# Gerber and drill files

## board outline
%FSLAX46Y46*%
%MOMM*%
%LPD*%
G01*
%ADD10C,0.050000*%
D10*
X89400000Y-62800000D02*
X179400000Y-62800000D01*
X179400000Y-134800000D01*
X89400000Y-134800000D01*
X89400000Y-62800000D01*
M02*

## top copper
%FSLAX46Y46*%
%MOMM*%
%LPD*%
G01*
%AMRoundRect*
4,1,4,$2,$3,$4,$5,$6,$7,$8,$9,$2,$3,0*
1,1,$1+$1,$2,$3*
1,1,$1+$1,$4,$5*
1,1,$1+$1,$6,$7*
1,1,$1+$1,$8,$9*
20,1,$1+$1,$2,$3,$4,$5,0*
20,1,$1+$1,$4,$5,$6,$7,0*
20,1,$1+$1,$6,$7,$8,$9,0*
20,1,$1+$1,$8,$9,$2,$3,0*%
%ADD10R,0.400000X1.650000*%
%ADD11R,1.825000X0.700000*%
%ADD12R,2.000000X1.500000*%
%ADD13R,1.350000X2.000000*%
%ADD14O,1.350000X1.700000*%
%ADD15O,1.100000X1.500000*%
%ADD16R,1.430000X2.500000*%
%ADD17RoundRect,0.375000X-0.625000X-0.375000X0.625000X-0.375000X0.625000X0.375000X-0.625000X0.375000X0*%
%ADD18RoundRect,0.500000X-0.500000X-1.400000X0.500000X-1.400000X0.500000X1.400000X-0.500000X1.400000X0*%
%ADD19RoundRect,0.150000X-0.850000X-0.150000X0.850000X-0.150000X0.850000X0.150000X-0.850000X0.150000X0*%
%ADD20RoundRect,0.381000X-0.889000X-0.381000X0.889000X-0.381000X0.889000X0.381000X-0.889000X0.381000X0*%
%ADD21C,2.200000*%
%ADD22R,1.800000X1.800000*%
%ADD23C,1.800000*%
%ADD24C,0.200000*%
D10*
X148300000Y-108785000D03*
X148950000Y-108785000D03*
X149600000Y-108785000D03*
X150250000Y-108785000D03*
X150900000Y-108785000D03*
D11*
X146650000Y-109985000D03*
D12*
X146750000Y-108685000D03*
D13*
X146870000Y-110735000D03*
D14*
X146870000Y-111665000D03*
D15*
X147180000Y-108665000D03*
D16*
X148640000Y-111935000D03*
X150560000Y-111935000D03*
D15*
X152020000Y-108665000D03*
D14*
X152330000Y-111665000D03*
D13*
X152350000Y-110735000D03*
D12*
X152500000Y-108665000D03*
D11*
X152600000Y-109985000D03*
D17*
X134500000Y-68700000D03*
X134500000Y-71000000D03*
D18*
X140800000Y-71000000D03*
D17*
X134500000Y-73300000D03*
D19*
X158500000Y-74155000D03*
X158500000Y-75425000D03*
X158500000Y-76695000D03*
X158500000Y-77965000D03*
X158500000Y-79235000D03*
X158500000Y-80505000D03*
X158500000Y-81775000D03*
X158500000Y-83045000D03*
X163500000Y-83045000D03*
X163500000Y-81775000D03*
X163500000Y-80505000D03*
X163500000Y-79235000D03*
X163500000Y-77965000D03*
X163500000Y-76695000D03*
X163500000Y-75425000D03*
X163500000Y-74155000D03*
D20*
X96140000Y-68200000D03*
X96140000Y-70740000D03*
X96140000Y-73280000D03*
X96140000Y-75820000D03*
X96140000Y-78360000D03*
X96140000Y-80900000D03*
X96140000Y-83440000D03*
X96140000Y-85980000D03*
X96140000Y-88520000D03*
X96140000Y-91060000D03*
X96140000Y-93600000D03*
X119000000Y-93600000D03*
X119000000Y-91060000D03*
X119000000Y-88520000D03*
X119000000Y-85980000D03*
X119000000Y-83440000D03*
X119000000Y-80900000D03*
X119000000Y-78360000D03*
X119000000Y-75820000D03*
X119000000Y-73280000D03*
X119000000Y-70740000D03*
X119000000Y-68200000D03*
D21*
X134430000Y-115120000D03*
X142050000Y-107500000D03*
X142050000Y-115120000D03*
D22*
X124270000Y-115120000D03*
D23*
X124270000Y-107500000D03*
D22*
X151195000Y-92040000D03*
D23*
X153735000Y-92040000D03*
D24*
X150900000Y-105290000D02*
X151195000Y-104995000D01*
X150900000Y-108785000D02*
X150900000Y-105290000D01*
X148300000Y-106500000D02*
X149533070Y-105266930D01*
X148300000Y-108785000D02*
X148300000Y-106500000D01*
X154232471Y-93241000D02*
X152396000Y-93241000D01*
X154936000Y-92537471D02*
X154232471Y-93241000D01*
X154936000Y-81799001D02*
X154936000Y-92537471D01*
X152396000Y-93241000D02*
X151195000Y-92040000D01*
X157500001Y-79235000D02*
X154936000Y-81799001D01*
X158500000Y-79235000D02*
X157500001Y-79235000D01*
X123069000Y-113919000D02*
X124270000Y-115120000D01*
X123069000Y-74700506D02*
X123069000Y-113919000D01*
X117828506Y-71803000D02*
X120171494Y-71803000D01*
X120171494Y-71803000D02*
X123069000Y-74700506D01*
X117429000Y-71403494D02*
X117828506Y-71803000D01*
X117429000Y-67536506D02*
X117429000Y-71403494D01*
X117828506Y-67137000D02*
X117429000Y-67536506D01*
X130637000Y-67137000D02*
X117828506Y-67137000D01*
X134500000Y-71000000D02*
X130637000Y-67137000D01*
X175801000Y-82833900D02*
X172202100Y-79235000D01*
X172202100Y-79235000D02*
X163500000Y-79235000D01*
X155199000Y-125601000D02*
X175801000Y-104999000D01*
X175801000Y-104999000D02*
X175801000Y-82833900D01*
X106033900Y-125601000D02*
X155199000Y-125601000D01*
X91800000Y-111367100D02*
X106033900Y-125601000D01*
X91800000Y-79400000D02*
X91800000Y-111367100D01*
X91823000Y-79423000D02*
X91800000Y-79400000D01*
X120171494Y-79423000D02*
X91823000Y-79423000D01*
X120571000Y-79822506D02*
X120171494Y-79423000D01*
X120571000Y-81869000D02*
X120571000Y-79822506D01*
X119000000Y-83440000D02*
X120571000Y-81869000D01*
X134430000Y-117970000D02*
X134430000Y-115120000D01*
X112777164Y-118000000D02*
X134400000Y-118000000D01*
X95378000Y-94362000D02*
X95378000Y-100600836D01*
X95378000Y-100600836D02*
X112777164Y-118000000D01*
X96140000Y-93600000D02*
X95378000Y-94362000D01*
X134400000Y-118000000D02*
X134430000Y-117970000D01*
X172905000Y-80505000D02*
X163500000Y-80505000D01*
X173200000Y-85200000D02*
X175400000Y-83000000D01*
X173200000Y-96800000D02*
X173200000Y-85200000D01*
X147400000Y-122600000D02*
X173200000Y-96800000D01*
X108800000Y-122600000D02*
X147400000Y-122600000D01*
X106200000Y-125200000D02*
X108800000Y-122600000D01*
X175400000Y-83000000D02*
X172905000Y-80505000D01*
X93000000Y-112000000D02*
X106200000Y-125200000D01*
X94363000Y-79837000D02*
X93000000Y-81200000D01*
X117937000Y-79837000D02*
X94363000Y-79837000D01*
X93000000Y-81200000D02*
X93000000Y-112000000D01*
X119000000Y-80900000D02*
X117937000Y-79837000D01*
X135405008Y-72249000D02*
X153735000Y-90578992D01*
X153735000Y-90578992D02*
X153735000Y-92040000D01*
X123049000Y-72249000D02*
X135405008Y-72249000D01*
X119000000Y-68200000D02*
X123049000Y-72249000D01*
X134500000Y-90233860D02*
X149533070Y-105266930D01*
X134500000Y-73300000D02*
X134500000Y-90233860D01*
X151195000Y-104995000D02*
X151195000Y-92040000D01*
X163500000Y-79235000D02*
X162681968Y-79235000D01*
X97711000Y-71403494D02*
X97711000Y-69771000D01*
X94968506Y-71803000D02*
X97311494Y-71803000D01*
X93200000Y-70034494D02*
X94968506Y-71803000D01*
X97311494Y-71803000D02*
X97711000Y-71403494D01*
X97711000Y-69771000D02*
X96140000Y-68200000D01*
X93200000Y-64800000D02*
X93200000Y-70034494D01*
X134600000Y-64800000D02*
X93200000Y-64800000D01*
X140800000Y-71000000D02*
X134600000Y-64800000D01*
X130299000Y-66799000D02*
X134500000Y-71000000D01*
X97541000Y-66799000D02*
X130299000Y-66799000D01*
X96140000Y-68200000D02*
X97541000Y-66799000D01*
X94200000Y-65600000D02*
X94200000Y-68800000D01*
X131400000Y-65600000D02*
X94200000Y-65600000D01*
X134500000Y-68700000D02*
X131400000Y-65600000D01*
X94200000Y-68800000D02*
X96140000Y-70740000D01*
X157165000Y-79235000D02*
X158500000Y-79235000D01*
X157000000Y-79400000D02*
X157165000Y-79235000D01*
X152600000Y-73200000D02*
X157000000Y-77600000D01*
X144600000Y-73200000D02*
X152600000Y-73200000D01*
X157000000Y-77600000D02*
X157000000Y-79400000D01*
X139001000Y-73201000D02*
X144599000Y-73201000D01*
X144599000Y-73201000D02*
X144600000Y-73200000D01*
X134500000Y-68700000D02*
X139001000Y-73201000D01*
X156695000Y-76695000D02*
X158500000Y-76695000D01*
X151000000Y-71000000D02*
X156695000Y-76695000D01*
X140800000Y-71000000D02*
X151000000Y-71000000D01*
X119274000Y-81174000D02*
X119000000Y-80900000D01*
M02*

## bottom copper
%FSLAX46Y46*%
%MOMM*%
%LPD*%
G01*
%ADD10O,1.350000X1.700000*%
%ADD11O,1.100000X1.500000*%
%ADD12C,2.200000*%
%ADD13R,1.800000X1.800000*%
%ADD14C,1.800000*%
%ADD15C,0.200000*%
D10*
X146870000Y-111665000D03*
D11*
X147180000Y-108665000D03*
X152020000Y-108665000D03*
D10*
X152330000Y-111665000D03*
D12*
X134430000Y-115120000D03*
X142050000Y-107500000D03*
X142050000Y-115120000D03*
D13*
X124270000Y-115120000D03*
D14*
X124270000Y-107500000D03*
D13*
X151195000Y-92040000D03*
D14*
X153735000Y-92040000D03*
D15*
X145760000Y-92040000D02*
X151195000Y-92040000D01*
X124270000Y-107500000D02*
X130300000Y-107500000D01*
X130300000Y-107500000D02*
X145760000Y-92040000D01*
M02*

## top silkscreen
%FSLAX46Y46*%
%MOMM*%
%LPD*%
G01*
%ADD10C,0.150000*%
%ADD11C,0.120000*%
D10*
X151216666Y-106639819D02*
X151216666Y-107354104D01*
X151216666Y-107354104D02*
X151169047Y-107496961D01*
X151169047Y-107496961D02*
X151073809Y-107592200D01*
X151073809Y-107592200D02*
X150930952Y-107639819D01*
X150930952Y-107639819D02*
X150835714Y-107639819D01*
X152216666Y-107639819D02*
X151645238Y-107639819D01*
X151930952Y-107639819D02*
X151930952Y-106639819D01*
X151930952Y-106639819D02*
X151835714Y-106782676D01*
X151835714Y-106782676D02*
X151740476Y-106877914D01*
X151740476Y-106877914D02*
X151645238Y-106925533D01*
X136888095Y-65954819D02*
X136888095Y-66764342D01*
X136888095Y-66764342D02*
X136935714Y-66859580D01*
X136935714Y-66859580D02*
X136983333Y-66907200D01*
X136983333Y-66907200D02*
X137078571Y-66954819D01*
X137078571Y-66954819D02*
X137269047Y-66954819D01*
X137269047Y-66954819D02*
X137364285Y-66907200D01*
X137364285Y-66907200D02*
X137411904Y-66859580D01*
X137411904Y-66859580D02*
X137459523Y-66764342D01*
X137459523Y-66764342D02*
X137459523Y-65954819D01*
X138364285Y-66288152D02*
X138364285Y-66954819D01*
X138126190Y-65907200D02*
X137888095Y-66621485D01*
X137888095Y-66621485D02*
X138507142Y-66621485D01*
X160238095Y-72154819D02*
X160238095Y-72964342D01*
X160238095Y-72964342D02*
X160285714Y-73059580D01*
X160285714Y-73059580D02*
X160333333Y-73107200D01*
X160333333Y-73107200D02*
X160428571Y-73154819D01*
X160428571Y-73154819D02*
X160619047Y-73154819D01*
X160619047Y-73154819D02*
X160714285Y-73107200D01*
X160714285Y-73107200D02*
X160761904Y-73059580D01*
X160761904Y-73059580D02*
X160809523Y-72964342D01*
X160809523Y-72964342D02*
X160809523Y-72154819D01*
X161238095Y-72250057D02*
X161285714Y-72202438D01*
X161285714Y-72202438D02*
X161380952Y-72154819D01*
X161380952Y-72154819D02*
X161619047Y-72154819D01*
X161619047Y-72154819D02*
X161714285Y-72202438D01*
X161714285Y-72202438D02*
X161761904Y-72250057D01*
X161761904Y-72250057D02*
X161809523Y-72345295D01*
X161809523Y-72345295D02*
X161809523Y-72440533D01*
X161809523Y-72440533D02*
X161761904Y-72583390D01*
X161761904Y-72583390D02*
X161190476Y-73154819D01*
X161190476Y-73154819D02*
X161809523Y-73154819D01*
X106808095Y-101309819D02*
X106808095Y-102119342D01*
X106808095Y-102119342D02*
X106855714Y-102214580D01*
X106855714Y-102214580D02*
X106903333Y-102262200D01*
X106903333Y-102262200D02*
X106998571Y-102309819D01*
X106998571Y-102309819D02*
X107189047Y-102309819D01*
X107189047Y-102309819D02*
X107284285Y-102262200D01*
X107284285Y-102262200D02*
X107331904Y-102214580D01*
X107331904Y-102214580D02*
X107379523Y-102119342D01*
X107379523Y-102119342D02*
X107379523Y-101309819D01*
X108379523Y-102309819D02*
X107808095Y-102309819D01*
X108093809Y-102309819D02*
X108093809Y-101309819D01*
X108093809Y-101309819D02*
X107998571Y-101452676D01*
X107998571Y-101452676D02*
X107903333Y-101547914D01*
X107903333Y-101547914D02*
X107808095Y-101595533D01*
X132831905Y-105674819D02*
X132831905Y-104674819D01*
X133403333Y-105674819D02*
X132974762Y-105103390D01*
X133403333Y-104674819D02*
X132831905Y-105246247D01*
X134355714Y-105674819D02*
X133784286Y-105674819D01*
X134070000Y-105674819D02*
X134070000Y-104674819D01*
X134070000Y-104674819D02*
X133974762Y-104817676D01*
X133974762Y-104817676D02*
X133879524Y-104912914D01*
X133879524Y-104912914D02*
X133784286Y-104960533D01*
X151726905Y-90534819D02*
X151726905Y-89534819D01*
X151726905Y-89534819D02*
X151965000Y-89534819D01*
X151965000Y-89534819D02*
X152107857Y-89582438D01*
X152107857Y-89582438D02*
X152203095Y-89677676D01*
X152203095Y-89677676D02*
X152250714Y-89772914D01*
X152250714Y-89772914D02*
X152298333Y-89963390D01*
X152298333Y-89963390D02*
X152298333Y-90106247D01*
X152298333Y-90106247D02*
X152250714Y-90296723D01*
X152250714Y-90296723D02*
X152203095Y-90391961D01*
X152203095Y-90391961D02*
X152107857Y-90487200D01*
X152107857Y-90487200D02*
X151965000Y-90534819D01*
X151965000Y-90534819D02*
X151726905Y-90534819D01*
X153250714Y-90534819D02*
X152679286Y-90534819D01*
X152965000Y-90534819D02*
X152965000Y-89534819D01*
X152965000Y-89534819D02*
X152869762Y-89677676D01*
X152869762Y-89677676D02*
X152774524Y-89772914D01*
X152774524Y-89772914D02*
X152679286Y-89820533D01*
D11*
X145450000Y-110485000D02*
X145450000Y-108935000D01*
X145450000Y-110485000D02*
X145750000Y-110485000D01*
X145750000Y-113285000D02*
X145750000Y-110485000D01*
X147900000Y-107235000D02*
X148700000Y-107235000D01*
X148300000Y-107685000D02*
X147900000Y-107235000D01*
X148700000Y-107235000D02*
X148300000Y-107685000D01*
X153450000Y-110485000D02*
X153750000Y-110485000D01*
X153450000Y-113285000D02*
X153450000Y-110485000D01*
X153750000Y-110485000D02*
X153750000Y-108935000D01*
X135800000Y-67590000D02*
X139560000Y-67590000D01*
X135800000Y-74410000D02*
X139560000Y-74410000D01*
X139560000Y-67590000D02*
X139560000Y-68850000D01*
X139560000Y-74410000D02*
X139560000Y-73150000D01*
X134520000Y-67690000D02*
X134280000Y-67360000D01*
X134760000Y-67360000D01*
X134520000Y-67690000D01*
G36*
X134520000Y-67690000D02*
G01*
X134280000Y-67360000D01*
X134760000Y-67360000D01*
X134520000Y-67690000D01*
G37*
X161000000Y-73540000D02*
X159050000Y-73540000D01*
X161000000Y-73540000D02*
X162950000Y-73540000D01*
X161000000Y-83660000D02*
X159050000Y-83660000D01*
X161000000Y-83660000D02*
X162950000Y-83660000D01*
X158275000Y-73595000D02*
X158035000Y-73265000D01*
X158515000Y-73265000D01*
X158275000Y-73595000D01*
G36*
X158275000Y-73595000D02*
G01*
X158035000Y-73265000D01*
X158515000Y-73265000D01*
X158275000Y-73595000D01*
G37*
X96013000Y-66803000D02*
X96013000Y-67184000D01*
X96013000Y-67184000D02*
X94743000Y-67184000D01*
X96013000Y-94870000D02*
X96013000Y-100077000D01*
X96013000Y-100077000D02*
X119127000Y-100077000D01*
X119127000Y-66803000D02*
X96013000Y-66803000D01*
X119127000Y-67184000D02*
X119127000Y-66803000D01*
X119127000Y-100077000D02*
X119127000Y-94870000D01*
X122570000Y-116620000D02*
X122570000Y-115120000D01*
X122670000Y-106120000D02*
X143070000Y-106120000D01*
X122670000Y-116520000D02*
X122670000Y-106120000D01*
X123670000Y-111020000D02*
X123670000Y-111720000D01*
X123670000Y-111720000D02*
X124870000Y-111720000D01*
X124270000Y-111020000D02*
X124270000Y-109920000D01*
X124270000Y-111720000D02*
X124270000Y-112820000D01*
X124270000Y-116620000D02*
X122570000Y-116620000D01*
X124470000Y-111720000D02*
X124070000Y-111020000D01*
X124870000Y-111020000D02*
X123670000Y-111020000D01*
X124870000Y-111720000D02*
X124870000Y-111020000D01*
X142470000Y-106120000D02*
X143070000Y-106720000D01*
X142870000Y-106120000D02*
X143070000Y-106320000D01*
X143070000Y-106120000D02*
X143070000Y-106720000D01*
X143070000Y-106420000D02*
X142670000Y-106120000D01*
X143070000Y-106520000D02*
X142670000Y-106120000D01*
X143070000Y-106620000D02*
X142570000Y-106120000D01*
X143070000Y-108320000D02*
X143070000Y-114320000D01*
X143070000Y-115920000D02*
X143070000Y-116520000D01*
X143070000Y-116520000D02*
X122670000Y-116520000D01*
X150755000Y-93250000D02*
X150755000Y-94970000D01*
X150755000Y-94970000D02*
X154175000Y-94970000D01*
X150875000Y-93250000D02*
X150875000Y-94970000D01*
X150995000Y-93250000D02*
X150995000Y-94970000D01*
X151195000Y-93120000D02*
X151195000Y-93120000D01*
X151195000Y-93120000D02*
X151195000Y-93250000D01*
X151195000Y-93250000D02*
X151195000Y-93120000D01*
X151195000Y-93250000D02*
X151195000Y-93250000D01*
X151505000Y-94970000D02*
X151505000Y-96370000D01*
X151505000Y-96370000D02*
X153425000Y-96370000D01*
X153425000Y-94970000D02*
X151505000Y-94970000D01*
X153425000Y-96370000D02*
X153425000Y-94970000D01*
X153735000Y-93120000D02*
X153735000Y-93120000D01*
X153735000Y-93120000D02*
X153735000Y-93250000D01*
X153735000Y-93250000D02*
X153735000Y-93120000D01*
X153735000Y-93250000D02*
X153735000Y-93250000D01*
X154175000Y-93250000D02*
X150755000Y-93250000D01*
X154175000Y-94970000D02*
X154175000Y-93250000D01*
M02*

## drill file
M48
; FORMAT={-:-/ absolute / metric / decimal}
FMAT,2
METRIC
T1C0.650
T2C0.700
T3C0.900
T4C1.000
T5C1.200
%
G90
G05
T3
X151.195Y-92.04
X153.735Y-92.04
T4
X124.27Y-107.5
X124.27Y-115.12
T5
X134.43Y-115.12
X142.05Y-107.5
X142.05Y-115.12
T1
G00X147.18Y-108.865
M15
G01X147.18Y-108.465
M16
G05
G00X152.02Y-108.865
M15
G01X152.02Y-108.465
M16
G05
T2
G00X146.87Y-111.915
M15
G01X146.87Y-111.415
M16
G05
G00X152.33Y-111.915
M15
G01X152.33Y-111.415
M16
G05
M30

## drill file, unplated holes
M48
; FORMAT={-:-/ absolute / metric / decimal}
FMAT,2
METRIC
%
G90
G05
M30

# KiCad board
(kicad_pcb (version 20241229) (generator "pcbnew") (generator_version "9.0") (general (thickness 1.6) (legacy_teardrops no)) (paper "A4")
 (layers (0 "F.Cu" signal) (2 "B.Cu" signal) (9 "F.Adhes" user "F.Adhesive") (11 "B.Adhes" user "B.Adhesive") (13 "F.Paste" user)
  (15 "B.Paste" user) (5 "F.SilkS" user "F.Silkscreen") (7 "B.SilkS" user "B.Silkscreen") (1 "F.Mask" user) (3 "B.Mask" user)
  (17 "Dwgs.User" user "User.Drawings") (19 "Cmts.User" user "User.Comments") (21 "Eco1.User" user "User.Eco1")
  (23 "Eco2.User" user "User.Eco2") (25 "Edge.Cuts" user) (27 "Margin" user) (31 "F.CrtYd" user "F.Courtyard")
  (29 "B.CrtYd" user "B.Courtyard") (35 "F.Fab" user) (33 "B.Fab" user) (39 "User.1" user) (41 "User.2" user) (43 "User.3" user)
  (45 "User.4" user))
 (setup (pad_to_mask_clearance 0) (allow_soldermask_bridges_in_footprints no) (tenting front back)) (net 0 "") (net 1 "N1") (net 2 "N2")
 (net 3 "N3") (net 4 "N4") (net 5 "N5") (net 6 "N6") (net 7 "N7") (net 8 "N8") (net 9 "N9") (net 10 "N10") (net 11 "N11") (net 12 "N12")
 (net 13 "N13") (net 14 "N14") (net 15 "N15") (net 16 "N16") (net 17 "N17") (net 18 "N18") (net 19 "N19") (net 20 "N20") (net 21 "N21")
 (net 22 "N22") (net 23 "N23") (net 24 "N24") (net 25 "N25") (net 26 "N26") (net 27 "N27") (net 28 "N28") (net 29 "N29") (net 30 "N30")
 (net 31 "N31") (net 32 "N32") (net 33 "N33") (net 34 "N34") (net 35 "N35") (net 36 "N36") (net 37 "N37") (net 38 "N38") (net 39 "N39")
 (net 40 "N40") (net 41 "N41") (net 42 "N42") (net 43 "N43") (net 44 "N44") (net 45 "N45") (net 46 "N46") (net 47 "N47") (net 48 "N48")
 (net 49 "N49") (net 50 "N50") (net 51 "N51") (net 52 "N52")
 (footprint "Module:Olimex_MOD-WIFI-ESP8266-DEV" (layer "F.Cu") (at 107.57 80.9)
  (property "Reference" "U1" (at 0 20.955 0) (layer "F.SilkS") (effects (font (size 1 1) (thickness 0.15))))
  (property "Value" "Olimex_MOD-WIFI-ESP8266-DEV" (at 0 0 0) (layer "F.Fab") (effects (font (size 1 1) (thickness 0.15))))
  (fp_line (start -11.557 -14.097) (end -11.557 -13.716) (stroke (width 0.12) (type solid)) (layer "F.SilkS"))
  (fp_line (start -11.557 -13.716) (end -12.827 -13.716) (stroke (width 0.12) (type solid)) (layer "F.SilkS"))
  (fp_line (start -11.557 13.97) (end -11.557 19.177) (stroke (width 0.12) (type solid)) (layer "F.SilkS"))
  (fp_line (start -11.557 19.177) (end 11.557 19.177) (stroke (width 0.12) (type solid)) (layer "F.SilkS"))
  (fp_line (start 11.557 -14.097) (end -11.557 -14.097) (stroke (width 0.12) (type solid)) (layer "F.SilkS"))
  (fp_line (start 11.557 -13.716) (end 11.557 -14.097) (stroke (width 0.12) (type solid)) (layer "F.SilkS"))
  (fp_line (start 11.557 19.177) (end 11.557 13.97) (stroke (width 0.12) (type solid)) (layer "F.SilkS"))
  (pad "1" smd roundrect (at -11.43 -12.7) (size 2.54 1.524) (layers "F.Cu" "F.Mask" "F.Paste") (roundrect_rratio 0.25) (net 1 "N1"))
  (pad "2" smd roundrect (at -11.43 -10.16) (size 2.54 1.524) (layers "F.Cu" "F.Mask" "F.Paste") (roundrect_rratio 0.25) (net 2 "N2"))
  (pad "3" smd roundrect (at -11.43 -7.62) (size 2.54 1.524) (layers "F.Cu" "F.Mask" "F.Paste") (roundrect_rratio 0.25) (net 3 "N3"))
  (pad "4" smd roundrect (at -11.43 -5.08) (size 2.54 1.524) (layers "F.Cu" "F.Mask" "F.Paste") (roundrect_rratio 0.25) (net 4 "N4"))
  (pad "5" smd roundrect (at -11.43 -2.54) (size 2.54 1.524) (layers "F.Cu" "F.Mask" "F.Paste") (roundrect_rratio 0.25) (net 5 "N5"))
  (pad "6" smd roundrect (at -11.43 0) (size 2.54 1.524) (layers "F.Cu" "F.Mask" "F.Paste") (roundrect_rratio 0.25) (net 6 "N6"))
  (pad "7" smd roundrect (at -11.43 2.54) (size 2.54 1.524) (layers "F.Cu" "F.Mask" "F.Paste") (roundrect_rratio 0.25) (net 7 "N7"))
  (pad "8" smd roundrect (at -11.43 5.08) (size 2.54 1.524) (layers "F.Cu" "F.Mask" "F.Paste") (roundrect_rratio 0.25) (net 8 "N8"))
  (pad "9" smd roundrect (at -11.43 7.62) (size 2.54 1.524) (layers "F.Cu" "F.Mask" "F.Paste") (roundrect_rratio 0.25) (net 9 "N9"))
  (pad "10" smd roundrect (at -11.43 10.16) (size 2.54 1.524) (layers "F.Cu" "F.Mask" "F.Paste") (roundrect_rratio 0.25) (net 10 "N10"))
  (pad "11" smd roundrect (at -11.43 12.7) (size 2.54 1.524) (layers "F.Cu" "F.Mask" "F.Paste") (roundrect_rratio 0.25) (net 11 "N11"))
  (pad "12" smd roundrect (at 11.43 12.7) (size 2.54 1.524) (layers "F.Cu" "F.Mask" "F.Paste") (roundrect_rratio 0.25) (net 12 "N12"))
  (pad "13" smd roundrect (at 11.43 10.16) (size 2.54 1.524) (layers "F.Cu" "F.Mask" "F.Paste") (roundrect_rratio 0.25) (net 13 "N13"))
  (pad "14" smd roundrect (at 11.43 7.62) (size 2.54 1.524) (layers "F.Cu" "F.Mask" "F.Paste") (roundrect_rratio 0.25) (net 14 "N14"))
  (pad "15" smd roundrect (at 11.43 5.08) (size 2.54 1.524) (layers "F.Cu" "F.Mask" "F.Paste") (roundrect_rratio 0.25) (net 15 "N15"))
  (pad "16" smd roundrect (at 11.43 2.54) (size 2.54 1.524) (layers "F.Cu" "F.Mask" "F.Paste") (roundrect_rratio 0.25) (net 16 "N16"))
  (pad "17" smd roundrect (at 11.43 0) (size 2.54 1.524) (layers "F.Cu" "F.Mask" "F.Paste") (roundrect_rratio 0.25) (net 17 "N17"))
  (pad "18" smd roundrect (at 11.43 -2.54) (size 2.54 1.524) (layers "F.Cu" "F.Mask" "F.Paste") (roundrect_rratio 0.25) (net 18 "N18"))
  (pad "19" smd roundrect (at 11.43 -5.08) (size 2.54 1.524) (layers "F.Cu" "F.Mask" "F.Paste") (roundrect_rratio 0.25) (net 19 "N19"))
  (pad "20" smd roundrect (at 11.43 -7.62) (size 2.54 1.524) (layers "F.Cu" "F.Mask" "F.Paste") (roundrect_rratio 0.25) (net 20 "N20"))
  (pad "21" smd roundrect (at 11.43 -10.16) (size 2.54 1.524) (layers "F.Cu" "F.Mask" "F.Paste") (roundrect_rratio 0.25) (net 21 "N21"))
  (pad "22" smd roundrect (at 11.43 -12.7) (size 2.54 1.524) (layers "F.Cu" "F.Mask" "F.Paste") (roundrect_rratio 0.25) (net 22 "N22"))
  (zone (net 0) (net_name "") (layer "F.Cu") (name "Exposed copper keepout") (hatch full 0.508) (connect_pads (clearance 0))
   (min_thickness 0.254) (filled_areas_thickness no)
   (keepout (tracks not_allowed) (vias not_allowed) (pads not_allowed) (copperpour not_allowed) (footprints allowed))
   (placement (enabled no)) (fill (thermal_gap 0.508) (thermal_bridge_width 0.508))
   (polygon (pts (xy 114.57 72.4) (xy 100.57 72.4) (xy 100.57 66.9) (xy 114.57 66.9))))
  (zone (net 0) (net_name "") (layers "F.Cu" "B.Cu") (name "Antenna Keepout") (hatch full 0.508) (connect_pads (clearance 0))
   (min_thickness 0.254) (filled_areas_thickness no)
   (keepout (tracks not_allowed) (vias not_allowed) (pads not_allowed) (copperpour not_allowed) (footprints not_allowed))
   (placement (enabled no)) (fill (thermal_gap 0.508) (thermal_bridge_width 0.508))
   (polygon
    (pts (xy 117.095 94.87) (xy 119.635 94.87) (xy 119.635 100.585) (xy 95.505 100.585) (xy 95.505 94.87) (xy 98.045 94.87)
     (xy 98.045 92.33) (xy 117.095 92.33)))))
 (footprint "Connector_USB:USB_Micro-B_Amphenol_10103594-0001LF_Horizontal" (layer "F.Cu") (at 149.625 110.55)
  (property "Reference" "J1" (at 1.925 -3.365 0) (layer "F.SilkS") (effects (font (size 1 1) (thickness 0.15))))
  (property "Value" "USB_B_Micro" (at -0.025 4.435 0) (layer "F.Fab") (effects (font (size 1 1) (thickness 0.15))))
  (fp_line (start -4.175 -0.065) (end -4.175 -1.615) (stroke (width 0.12) (type solid)) (layer "F.SilkS"))
  (fp_line (start -4.175 -0.065) (end -3.875 -0.065) (stroke (width 0.12) (type solid)) (layer "F.SilkS"))
  (fp_line (start -3.875 2.735) (end -3.875 -0.065) (stroke (width 0.12) (type solid)) (layer "F.SilkS"))
  (fp_line (start -1.725 -3.315) (end -0.925 -3.315) (stroke (width 0.12) (type solid)) (layer "F.SilkS"))
  (fp_line (start -1.325 -2.865) (end -1.725 -3.315) (stroke (width 0.12) (type solid)) (layer "F.SilkS"))
  (fp_line (start -0.925 -3.315) (end -1.325 -2.865) (stroke (width 0.12) (type solid)) (layer "F.SilkS"))
  (fp_line (start 3.825 -0.065) (end 4.125 -0.065) (stroke (width 0.12) (type solid)) (layer "F.SilkS"))
  (fp_line (start 3.825 2.735) (end 3.825 -0.065) (stroke (width 0.12) (type solid)) (layer "F.SilkS"))
  (fp_line (start 4.125 -0.065) (end 4.125 -1.615) (stroke (width 0.12) (type solid)) (layer "F.SilkS"))
  (pad "1" smd rect (at -1.325 -1.765 90) (size 1.65 0.4) (layers "F.Cu" "F.Mask" "F.Paste") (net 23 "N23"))
  (pad "2" smd rect (at -0.675 -1.765 90) (size 1.65 0.4) (layers "F.Cu" "F.Mask" "F.Paste") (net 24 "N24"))
  (pad "3" smd rect (at -0.025 -1.765 90) (size 1.65 0.4) (layers "F.Cu" "F.Mask" "F.Paste") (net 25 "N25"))
  (pad "4" smd rect (at 0.625 -1.765 90) (size 1.65 0.4) (layers "F.Cu" "F.Mask" "F.Paste") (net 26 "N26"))
  (pad "5" smd rect (at 1.275 -1.765 90) (size 1.65 0.4) (layers "F.Cu" "F.Mask" "F.Paste") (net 2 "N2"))
  (pad "6" smd rect (at -2.975 -0.565) (size 1.825 0.7) (layers "F.Cu" "F.Mask" "F.Paste") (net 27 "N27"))
  (pad "6" smd rect (at -2.875 -1.865) (size 2 1.5) (layers "F.Cu" "F.Mask" "F.Paste") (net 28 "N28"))
  (pad "6" smd rect (at -2.755 0.185) (size 1.35 2) (layers "F.Cu" "F.Mask" "F.Paste") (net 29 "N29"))
  (pad "6" thru_hole oval (at -2.755 1.115 90) (size 1.7 1.35) (drill oval 1.2 0.7) (layers "*.Cu" "*.Mask") (remove_unused_layers no)
   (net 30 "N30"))
  (pad "6" thru_hole oval (at -2.445 -1.885 90) (size 1.5 1.1) (drill oval 1.05 0.65) (layers "*.Cu" "*.Mask") (remove_unused_layers no)
   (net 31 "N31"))
  (pad "6" smd rect (at -0.985 1.385 90) (size 2.5 1.43) (layers "F.Cu" "F.Mask" "F.Paste") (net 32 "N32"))
  (pad "6" smd rect (at 0.935 1.385 90) (size 2.5 1.43) (layers "F.Cu" "F.Mask" "F.Paste") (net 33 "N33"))
  (pad "6" thru_hole oval (at 2.395 -1.885 90) (size 1.5 1.1) (drill oval 1.05 0.65) (layers "*.Cu" "*.Mask") (remove_unused_layers no)
   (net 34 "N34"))
  (pad "6" thru_hole oval (at 2.705 1.115 90) (size 1.7 1.35) (drill oval 1.2 0.7) (layers "*.Cu" "*.Mask") (remove_unused_layers no)
   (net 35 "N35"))
  (pad "6" smd rect (at 2.725 0.185) (size 1.35 2) (layers "F.Cu" "F.Mask" "F.Paste") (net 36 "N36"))
  (pad "6" smd rect (at 2.875 -1.885) (size 2 1.5) (layers "F.Cu" "F.Mask" "F.Paste") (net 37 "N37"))
  (pad "6" smd rect (at 2.975 -0.565) (size 1.825 0.7) (layers "F.Cu" "F.Mask" "F.Paste") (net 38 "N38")))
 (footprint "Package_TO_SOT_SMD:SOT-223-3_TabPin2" (layer "F.Cu") (at 137.65 71)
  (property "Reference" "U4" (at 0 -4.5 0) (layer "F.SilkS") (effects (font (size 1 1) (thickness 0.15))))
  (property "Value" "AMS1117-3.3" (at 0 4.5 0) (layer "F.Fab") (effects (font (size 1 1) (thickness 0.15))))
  (fp_line (start -1.85 -3.41) (end 1.91 -3.41) (stroke (width 0.12) (type solid)) (layer "F.SilkS"))
  (fp_line (start -1.85 3.41) (end 1.91 3.41) (stroke (width 0.12) (type solid)) (layer "F.SilkS"))
  (fp_line (start 1.91 -3.41) (end 1.91 -2.15) (stroke (width 0.12) (type solid)) (layer "F.SilkS"))
  (fp_line (start 1.91 3.41) (end 1.91 2.15) (stroke (width 0.12) (type solid)) (layer "F.SilkS"))
  (fp_poly
   (pts (xy -3.13 -3.31) (xy -3.37 -3.64) (xy -2.89 -3.64) (xy -3.13 -3.31)) (stroke (width 0.12) (type solid)) (fill yes) (layer "F.SilkS"))
  (pad "1" smd roundrect (at -3.15 -2.3) (size 2 1.5) (layers "F.Cu" "F.Mask" "F.Paste") (roundrect_rratio 0.25) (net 2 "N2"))
  (pad "2" smd roundrect (at -3.15 0) (size 2 1.5) (layers "F.Cu" "F.Mask" "F.Paste") (roundrect_rratio 0.25) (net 1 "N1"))
  (pad "2" smd roundrect (at 3.15 0) (size 2 3.8) (layers "F.Cu" "F.Mask" "F.Paste") (roundrect_rratio 0.25) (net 1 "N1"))
  (pad "3" smd roundrect (at -3.15 2.3) (size 2 1.5) (layers "F.Cu" "F.Mask" "F.Paste") (roundrect_rratio 0.25) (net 23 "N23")))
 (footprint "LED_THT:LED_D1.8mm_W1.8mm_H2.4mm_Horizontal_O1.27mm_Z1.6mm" (layer "F.Cu") (at 151.195 92.04)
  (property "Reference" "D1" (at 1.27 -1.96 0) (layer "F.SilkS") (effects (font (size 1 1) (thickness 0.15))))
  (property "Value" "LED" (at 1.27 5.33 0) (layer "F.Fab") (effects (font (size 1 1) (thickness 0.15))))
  (fp_line (start -0.44 1.21) (end -0.44 2.93) (stroke (width 0.12) (type solid)) (layer "F.SilkS"))
  (fp_line (start -0.44 2.93) (end 2.98 2.93) (stroke (width 0.12) (type solid)) (layer "F.SilkS"))
  (fp_line (start -0.32 1.21) (end -0.32 2.93) (stroke (width 0.12) (type solid)) (layer "F.SilkS"))
  (fp_line (start -0.2 1.21) (end -0.2 2.93) (stroke (width 0.12) (type solid)) (layer "F.SilkS"))
  (fp_line (start 0 1.08) (end 0 1.08) (stroke (width 0.12) (type solid)) (layer "F.SilkS"))
  (fp_line (start 0 1.08) (end 0 1.21) (stroke (width 0.12) (type solid)) (layer "F.SilkS"))
  (fp_line (start 0 1.21) (end 0 1.08) (stroke (width 0.12) (type solid)) (layer "F.SilkS"))
  (fp_line (start 0 1.21) (end 0 1.21) (stroke (width 0.12) (type solid)) (layer "F.SilkS"))
  (fp_line (start 0.31 2.93) (end 0.31 4.33) (stroke (width 0.12) (type solid)) (layer "F.SilkS"))
  (fp_line (start 0.31 4.33) (end 2.23 4.33) (stroke (width 0.12) (type solid)) (layer "F.SilkS"))
  (fp_line (start 2.23 2.93) (end 0.31 2.93) (stroke (width 0.12) (type solid)) (layer "F.SilkS"))
  (fp_line (start 2.23 4.33) (end 2.23 2.93) (stroke (width 0.12) (type solid)) (layer "F.SilkS"))
  (fp_line (start 2.54 1.08) (end 2.54 1.08) (stroke (width 0.12) (type solid)) (layer "F.SilkS"))
  (fp_line (start 2.54 1.08) (end 2.54 1.21) (stroke (width 0.12) (type solid)) (layer "F.SilkS"))
  (fp_line (start 2.54 1.21) (end 2.54 1.08) (stroke (width 0.12) (type solid)) (layer "F.SilkS"))
  (fp_line (start 2.54 1.21) (end 2.54 1.21) (stroke (width 0.12) (type solid)) (layer "F.SilkS"))
  (fp_line (start 2.98 1.21) (end -0.44 1.21) (stroke (width 0.12) (type solid)) (layer "F.SilkS"))
  (fp_line (start 2.98 2.93) (end 2.98 1.21) (stroke (width 0.12) (type solid)) (layer "F.SilkS"))
  (pad "1" thru_hole rect (at 0 0) (size 1.8 1.8) (drill 0.9) (layers "*.Cu" "*.Mask") (remove_unused_layers no) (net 2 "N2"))
  (pad "2" thru_hole circle (at 2.54 0) (size 1.8 1.8) (drill 0.9) (layers "*.Cu" "*.Mask") (remove_unused_layers no) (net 22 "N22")))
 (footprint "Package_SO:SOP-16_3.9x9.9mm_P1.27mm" (layer "F.Cu") (at 161 78.6)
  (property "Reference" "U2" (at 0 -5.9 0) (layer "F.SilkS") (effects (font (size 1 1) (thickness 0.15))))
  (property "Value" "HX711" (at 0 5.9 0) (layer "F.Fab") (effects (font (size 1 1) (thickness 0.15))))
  (fp_line (start 0 -5.06) (end -1.95 -5.06) (stroke (width 0.12) (type solid)) (layer "F.SilkS"))
  (fp_line (start 0 -5.06) (end 1.95 -5.06) (stroke (width 0.12) (type solid)) (layer "F.SilkS"))
  (fp_line (start 0 5.06) (end -1.95 5.06) (stroke (width 0.12) (type solid)) (layer "F.SilkS"))
  (fp_line (start 0 5.06) (end 1.95 5.06) (stroke (width 0.12) (type solid)) (layer "F.SilkS"))
  (fp_poly
   (pts (xy -2.725 -5.005) (xy -2.965 -5.335) (xy -2.485 -5.335) (xy -2.725 -5.005)) (stroke (width 0.12) (type solid)) (fill yes)
   (layer "F.SilkS"))
  (pad "1" smd roundrect (at -2.5 -4.445) (size 2 0.6) (layers "F.Cu" "F.Mask" "F.Paste") (roundrect_rratio 0.25) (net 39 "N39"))
  (pad "2" smd roundrect (at -2.5 -3.175) (size 2 0.6) (layers "F.Cu" "F.Mask" "F.Paste") (roundrect_rratio 0.25) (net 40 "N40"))
  (pad "3" smd roundrect (at -2.5 -1.905) (size 2 0.6) (layers "F.Cu" "F.Mask" "F.Paste") (roundrect_rratio 0.25) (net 1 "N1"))
  (pad "4" smd roundrect (at -2.5 -0.635) (size 2 0.6) (layers "F.Cu" "F.Mask" "F.Paste") (roundrect_rratio 0.25) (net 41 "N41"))
  (pad "5" smd roundrect (at -2.5 0.635) (size 2 0.6) (layers "F.Cu" "F.Mask" "F.Paste") (roundrect_rratio 0.25) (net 2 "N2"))
  (pad "6" smd roundrect (at -2.5 1.905) (size 2 0.6) (layers "F.Cu" "F.Mask" "F.Paste") (roundrect_rratio 0.25) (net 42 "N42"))
  (pad "7" smd roundrect (at -2.5 3.175) (size 2 0.6) (layers "F.Cu" "F.Mask" "F.Paste") (roundrect_rratio 0.25) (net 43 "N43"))
  (pad "8" smd roundrect (at -2.5 4.445) (size 2 0.6) (layers "F.Cu" "F.Mask" "F.Paste") (roundrect_rratio 0.25) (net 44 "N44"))
  (pad "9" smd roundrect (at 2.5 4.445) (size 2 0.6) (layers "F.Cu" "F.Mask" "F.Paste") (roundrect_rratio 0.25) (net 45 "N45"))
  (pad "10" smd roundrect (at 2.5 3.175) (size 2 0.6) (layers "F.Cu" "F.Mask" "F.Paste") (roundrect_rratio 0.25) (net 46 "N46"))
  (pad "11" smd roundrect (at 2.5 1.905) (size 2 0.6) (layers "F.Cu" "F.Mask" "F.Paste") (roundrect_rratio 0.25) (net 17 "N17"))
  (pad "12" smd roundrect (at 2.5 0.635) (size 2 0.6) (layers "F.Cu" "F.Mask" "F.Paste") (roundrect_rratio 0.25) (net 16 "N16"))
  (pad "13" smd roundrect (at 2.5 -0.635) (size 2 0.6) (layers "F.Cu" "F.Mask" "F.Paste") (roundrect_rratio 0.25) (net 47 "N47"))
  (pad "14" smd roundrect (at 2.5 -1.905) (size 2 0.6) (layers "F.Cu" "F.Mask" "F.Paste") (roundrect_rratio 0.25) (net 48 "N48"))
  (pad "15" smd roundrect (at 2.5 -3.175) (size 2 0.6) (layers "F.Cu" "F.Mask" "F.Paste") (roundrect_rratio 0.25) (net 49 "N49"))
  (pad "16" smd roundrect (at 2.5 -4.445) (size 2 0.6) (layers "F.Cu" "F.Mask" "F.Paste") (roundrect_rratio 0.25) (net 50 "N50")))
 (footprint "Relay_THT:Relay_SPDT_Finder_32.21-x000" (layer "F.Cu") (at 124.27 115.12)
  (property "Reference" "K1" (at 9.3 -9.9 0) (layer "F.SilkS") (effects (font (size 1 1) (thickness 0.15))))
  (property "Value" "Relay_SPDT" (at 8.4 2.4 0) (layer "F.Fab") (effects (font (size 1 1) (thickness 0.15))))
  (fp_line (start -1.7 1.5) (end -1.7 0) (stroke (width 0.12) (type solid)) (layer "F.SilkS"))
  (fp_line (start -1.6 -9) (end 18.8 -9) (stroke (width 0.12) (type solid)) (layer "F.SilkS"))
  (fp_line (start -1.6 1.4) (end -1.6 -9) (stroke (width 0.12) (type solid)) (layer "F.SilkS"))
  (fp_line (start -0.6 -4.1) (end -0.6 -3.4) (stroke (width 0.12) (type solid)) (layer "F.SilkS"))
  (fp_line (start -0.6 -3.4) (end 0.6 -3.4) (stroke (width 0.12) (type solid)) (layer "F.SilkS"))
  (fp_line (start 0 -4.1) (end 0 -5.2) (stroke (width 0.12) (type solid)) (layer "F.SilkS"))
  (fp_line (start 0 -3.4) (end 0 -2.3) (stroke (width 0.12) (type solid)) (layer "F.SilkS"))
  (fp_line (start 0 1.5) (end -1.7 1.5) (stroke (width 0.12) (type solid)) (layer "F.SilkS"))
  (fp_line (start 0.2 -3.4) (end -0.2 -4.1) (stroke (width 0.12) (type solid)) (layer "F.SilkS"))
  (fp_line (start 0.6 -4.1) (end -0.6 -4.1) (stroke (width 0.12) (type solid)) (layer "F.SilkS"))
  (fp_line (start 0.6 -3.4) (end 0.6 -4.1) (stroke (width 0.12) (type solid)) (layer "F.SilkS"))
  (fp_line (start 18.2 -9) (end 18.8 -8.4) (stroke (width 0.12) (type solid)) (layer "F.SilkS"))
  (fp_line (start 18.6 -9) (end 18.8 -8.8) (stroke (width 0.12) (type solid)) (layer "F.SilkS"))
  (fp_line (start 18.8 -9) (end 18.8 -8.4) (stroke (width 0.12) (type solid)) (layer "F.SilkS"))
  (fp_line (start 18.8 -8.7) (end 18.4 -9) (stroke (width 0.12) (type solid)) (layer "F.SilkS"))
  (fp_line (start 18.8 -8.6) (end 18.4 -9) (stroke (width 0.12) (type solid)) (layer "F.SilkS"))
  (fp_line (start 18.8 -8.5) (end 18.3 -9) (stroke (width 0.12) (type solid)) (layer "F.SilkS"))
  (fp_line (start 18.8 -6.8) (end 18.8 -0.8) (stroke (width 0.12) (type solid)) (layer "F.SilkS"))
  (fp_line (start 18.8 0.8) (end 18.8 1.4) (stroke (width 0.12) (type solid)) (layer "F.SilkS"))
  (fp_line (start 18.8 1.4) (end -1.6 1.4) (stroke (width 0.12) (type solid)) (layer "F.SilkS"))
  (pad "11" thru_hole circle (at 10.16 0 90) (size 2.2 2.2) (drill 1.2) (layers "*.Cu" "*.Mask") (remove_unused_layers no) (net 11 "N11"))
  (pad "12" thru_hole circle (at 17.78 -7.62 90) (size 2.2 2.2) (drill 1.2) (layers "*.Cu" "*.Mask") (remove_unused_layers no)
   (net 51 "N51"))
  (pad "14" thru_hole circle (at 17.78 0 90) (size 2.2 2.2) (drill 1.2) (layers "*.Cu" "*.Mask") (remove_unused_layers no) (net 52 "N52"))
  (pad "A1" thru_hole rect (at 0 0 90) (size 1.8 1.8) (drill 1) (layers "*.Cu" "*.Mask") (remove_unused_layers no) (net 1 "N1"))
  (pad "A2" thru_hole circle (at 0 -7.62 90) (size 1.8 1.8) (drill 1) (layers "*.Cu" "*.Mask") (remove_unused_layers no) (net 2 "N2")))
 (gr_rect (start 89.4 62.8) (end 179.4 134.8) (stroke (width 0.05) (type default)) (fill no) (layer "Edge.Cuts"))
 (segment (start 123.049 72.249) (end 135.405008 72.249) (width 0.2) (layer "F.Cu") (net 22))
 (segment (start 153.735 90.578992) (end 153.735 92.04) (width 0.2) (layer "F.Cu") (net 22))
 (segment (start 135.405008 72.249) (end 153.735 90.578992) (width 0.2) (layer "F.Cu") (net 22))
 (segment (start 119 68.2) (end 123.049 72.249) (width 0.2) (layer "F.Cu") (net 22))
 (segment (start 131.4 65.6) (end 94.2 65.6) (width 0.2) (layer "F.Cu") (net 2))
 (segment (start 152.396 93.241) (end 151.195 92.04) (width 0.2) (layer "F.Cu") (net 2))
 (segment (start 134.5 68.7) (end 139.001 73.201) (width 0.2) (layer "F.Cu") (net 2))
 (segment (start 157 79.4) (end 157.165 79.235) (width 0.2) (layer "F.Cu") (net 2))
 (segment (start 94.2 65.6) (end 94.2 68.8) (width 0.2) (layer "F.Cu") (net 2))
 (segment (start 158.5 79.235) (end 157.500001 79.235) (width 0.2) (layer "F.Cu") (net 2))
 (segment (start 134.5 68.7) (end 131.4 65.6) (width 0.2) (layer "F.Cu") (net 2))
 (segment (start 94.2 68.8) (end 96.14 70.74) (width 0.2) (layer "F.Cu") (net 2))
 (segment (start 150.9 105.29) (end 151.195 104.995) (width 0.2) (layer "F.Cu") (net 2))
 (segment (start 150.9 108.785) (end 150.9 105.29) (width 0.2) (layer "F.Cu") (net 2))
 (segment (start 157 77.6) (end 157 79.4) (width 0.2) (layer "F.Cu") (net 2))
 (segment (start 144.6 73.2) (end 152.6 73.2) (width 0.2) (layer "F.Cu") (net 2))
 (segment (start 139.001 73.201) (end 144.599 73.201) (width 0.2) (layer "F.Cu") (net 2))
 (segment (start 154.232471 93.241) (end 152.396 93.241) (width 0.2) (layer "F.Cu") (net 2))
 (segment (start 154.936 81.799001) (end 154.936 92.537471) (width 0.2) (layer "F.Cu") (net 2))
 (segment (start 144.599 73.201) (end 144.6 73.2) (width 0.2) (layer "F.Cu") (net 2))
 (segment (start 157.500001 79.235) (end 154.936 81.799001) (width 0.2) (layer "F.Cu") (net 2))
 (segment (start 154.936 92.537471) (end 154.232471 93.241) (width 0.2) (layer "F.Cu") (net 2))
 (segment (start 151.195 104.995) (end 151.195 92.04) (width 0.2) (layer "F.Cu") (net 2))
 (segment (start 157.165 79.235) (end 158.5 79.235) (width 0.2) (layer "F.Cu") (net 2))
 (segment (start 152.6 73.2) (end 157 77.6) (width 0.2) (layer "F.Cu") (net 2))
 (segment (start 145.76 92.04) (end 151.195 92.04) (width 0.2) (layer "B.Cu") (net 2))
 (segment (start 130.3 107.5) (end 145.76 92.04) (width 0.2) (layer "B.Cu") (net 2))
 (segment (start 124.27 107.5) (end 130.3 107.5) (width 0.2) (layer "B.Cu") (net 2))
 (segment (start 134.5 73.3) (end 134.5 90.23386) (width 0.2) (layer "F.Cu") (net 23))
 (segment (start 148.3 108.785) (end 148.3 106.5) (width 0.2) (layer "F.Cu") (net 23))
 (segment (start 148.3 106.5) (end 149.53307 105.26693) (width 0.2) (layer "F.Cu") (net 23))
 (segment (start 134.5 90.23386) (end 149.53307 105.26693) (width 0.2) (layer "F.Cu") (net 23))
 (segment (start 96.14 93.6) (end 95.378 94.362) (width 0.2) (layer "F.Cu") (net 11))
 (segment (start 134.43 117.97) (end 134.43 115.12) (width 0.2) (layer "F.Cu") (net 11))
 (segment (start 95.378 100.600836) (end 112.777164 118) (width 0.2) (layer "F.Cu") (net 11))
 (segment (start 134.4 118) (end 134.43 117.97) (width 0.2) (layer "F.Cu") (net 11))
 (segment (start 95.378 94.362) (end 95.378 100.600836) (width 0.2) (layer "F.Cu") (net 11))
 (segment (start 112.777164 118) (end 134.4 118) (width 0.2) (layer "F.Cu") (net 11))
 (segment (start 140.8 71) (end 151 71) (width 0.2) (layer "F.Cu") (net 1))
 (segment (start 156.695 76.695) (end 158.5 76.695) (width 0.2) (layer "F.Cu") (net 1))
 (segment (start 123.069 113.919) (end 124.27 115.12) (width 0.2) (layer "F.Cu") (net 1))
 (segment (start 130.637 67.137) (end 117.828506 67.137) (width 0.2) (layer "F.Cu") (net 1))
 (segment (start 93.2 70.034494) (end 94.968506 71.803) (width 0.2) (layer "F.Cu") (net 1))
 (segment (start 97.711 71.403494) (end 97.711 69.771) (width 0.2) (layer "F.Cu") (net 1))
 (segment (start 117.828506 67.137) (end 117.429 67.536506) (width 0.2) (layer "F.Cu") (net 1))
 (segment (start 97.541 66.799) (end 130.299 66.799) (width 0.2) (layer "F.Cu") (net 1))
 (segment (start 97.711 69.771) (end 96.14 68.2) (width 0.2) (layer "F.Cu") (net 1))
 (segment (start 140.8 71) (end 134.6 64.8) (width 0.2) (layer "F.Cu") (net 1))
 (segment (start 151 71) (end 156.695 76.695) (width 0.2) (layer "F.Cu") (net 1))
 (segment (start 117.429 67.536506) (end 117.429 71.403494) (width 0.2) (layer "F.Cu") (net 1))
 (segment (start 123.069 74.700506) (end 123.069 113.919) (width 0.2) (layer "F.Cu") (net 1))
 (segment (start 94.968506 71.803) (end 97.311494 71.803) (width 0.2) (layer "F.Cu") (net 1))
 (segment (start 120.171494 71.803) (end 123.069 74.700506) (width 0.2) (layer "F.Cu") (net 1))
 (segment (start 134.5 71) (end 130.637 67.137) (width 0.2) (layer "F.Cu") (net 1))
 (segment (start 130.299 66.799) (end 134.5 71) (width 0.2) (layer "F.Cu") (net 1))
 (segment (start 96.14 68.2) (end 97.541 66.799) (width 0.2) (layer "F.Cu") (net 1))
 (segment (start 117.429 71.403494) (end 117.828506 71.803) (width 0.2) (layer "F.Cu") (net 1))
 (segment (start 93.2 64.8) (end 93.2 70.034494) (width 0.2) (layer "F.Cu") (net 1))
 (segment (start 117.828506 71.803) (end 120.171494 71.803) (width 0.2) (layer "F.Cu") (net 1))
 (segment (start 134.6 64.8) (end 93.2 64.8) (width 0.2) (layer "F.Cu") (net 1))
 (segment (start 97.311494 71.803) (end 97.711 71.403494) (width 0.2) (layer "F.Cu") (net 1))
 (segment (start 108.8 122.6) (end 147.4 122.6) (width 0.2) (layer "F.Cu") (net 17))
 (segment (start 173.2 96.8) (end 173.2 85.2) (width 0.2) (layer "F.Cu") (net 17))
 (segment (start 147.4 122.6) (end 173.2 96.8) (width 0.2) (layer "F.Cu") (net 17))
 (segment (start 172.905 80.505) (end 163.5 80.505) (width 0.2) (layer "F.Cu") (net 17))
 (segment (start 119.274 81.174) (end 119 80.9) (width 0.2) (layer "F.Cu") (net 17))
 (segment (start 93 81.2) (end 93 112) (width 0.2) (layer "F.Cu") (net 17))
 (segment (start 94.363 79.837) (end 93 81.2) (width 0.2) (layer "F.Cu") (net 17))
 (segment (start 106.2 125.2) (end 108.8 122.6) (width 0.2) (layer "F.Cu") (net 17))
 (segment (start 117.937 79.837) (end 94.363 79.837) (width 0.2) (layer "F.Cu") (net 17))
 (segment (start 119 80.9) (end 117.937 79.837) (width 0.2) (layer "F.Cu") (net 17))
 (segment (start 173.2 85.2) (end 175.4 83) (width 0.2) (layer "F.Cu") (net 17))
 (segment (start 93 112) (end 106.2 125.2) (width 0.2) (layer "F.Cu") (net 17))
 (segment (start 175.4 83) (end 172.905 80.505) (width 0.2) (layer "F.Cu") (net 17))
 (segment (start 175.801 104.999) (end 175.801 82.8339) (width 0.2) (layer "F.Cu") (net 16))
 (segment (start 91.8 111.3671) (end 106.0339 125.601) (width 0.2) (layer "F.Cu") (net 16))
 (segment (start 172.2021 79.235) (end 163.5 79.235) (width 0.2) (layer "F.Cu") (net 16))
 (segment (start 120.571 81.869) (end 120.571 79.822506) (width 0.2) (layer "F.Cu") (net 16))
 (segment (start 155.199 125.601) (end 175.801 104.999) (width 0.2) (layer "F.Cu") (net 16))
 (segment (start 106.0339 125.601) (end 155.199 125.601) (width 0.2) (layer "F.Cu") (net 16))
 (segment (start 120.571 79.822506) (end 120.171494 79.423) (width 0.2) (layer "F.Cu") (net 16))
 (segment (start 119 83.44) (end 120.571 81.869) (width 0.2) (layer "F.Cu") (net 16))
 (segment (start 175.801 82.8339) (end 172.2021 79.235) (width 0.2) (layer "F.Cu") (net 16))
 (segment (start 163.5 79.235) (end 162.681968 79.235) (width 0.2) (layer "F.Cu") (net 16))
 (segment (start 91.8 79.4) (end 91.8 111.3671) (width 0.2) (layer "F.Cu") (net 16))
 (segment (start 91.823 79.423) (end 91.8 79.4) (width 0.2) (layer "F.Cu") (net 16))
 (segment (start 120.171494 79.423) (end 91.823 79.423) (width 0.2) (layer "F.Cu") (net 16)))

